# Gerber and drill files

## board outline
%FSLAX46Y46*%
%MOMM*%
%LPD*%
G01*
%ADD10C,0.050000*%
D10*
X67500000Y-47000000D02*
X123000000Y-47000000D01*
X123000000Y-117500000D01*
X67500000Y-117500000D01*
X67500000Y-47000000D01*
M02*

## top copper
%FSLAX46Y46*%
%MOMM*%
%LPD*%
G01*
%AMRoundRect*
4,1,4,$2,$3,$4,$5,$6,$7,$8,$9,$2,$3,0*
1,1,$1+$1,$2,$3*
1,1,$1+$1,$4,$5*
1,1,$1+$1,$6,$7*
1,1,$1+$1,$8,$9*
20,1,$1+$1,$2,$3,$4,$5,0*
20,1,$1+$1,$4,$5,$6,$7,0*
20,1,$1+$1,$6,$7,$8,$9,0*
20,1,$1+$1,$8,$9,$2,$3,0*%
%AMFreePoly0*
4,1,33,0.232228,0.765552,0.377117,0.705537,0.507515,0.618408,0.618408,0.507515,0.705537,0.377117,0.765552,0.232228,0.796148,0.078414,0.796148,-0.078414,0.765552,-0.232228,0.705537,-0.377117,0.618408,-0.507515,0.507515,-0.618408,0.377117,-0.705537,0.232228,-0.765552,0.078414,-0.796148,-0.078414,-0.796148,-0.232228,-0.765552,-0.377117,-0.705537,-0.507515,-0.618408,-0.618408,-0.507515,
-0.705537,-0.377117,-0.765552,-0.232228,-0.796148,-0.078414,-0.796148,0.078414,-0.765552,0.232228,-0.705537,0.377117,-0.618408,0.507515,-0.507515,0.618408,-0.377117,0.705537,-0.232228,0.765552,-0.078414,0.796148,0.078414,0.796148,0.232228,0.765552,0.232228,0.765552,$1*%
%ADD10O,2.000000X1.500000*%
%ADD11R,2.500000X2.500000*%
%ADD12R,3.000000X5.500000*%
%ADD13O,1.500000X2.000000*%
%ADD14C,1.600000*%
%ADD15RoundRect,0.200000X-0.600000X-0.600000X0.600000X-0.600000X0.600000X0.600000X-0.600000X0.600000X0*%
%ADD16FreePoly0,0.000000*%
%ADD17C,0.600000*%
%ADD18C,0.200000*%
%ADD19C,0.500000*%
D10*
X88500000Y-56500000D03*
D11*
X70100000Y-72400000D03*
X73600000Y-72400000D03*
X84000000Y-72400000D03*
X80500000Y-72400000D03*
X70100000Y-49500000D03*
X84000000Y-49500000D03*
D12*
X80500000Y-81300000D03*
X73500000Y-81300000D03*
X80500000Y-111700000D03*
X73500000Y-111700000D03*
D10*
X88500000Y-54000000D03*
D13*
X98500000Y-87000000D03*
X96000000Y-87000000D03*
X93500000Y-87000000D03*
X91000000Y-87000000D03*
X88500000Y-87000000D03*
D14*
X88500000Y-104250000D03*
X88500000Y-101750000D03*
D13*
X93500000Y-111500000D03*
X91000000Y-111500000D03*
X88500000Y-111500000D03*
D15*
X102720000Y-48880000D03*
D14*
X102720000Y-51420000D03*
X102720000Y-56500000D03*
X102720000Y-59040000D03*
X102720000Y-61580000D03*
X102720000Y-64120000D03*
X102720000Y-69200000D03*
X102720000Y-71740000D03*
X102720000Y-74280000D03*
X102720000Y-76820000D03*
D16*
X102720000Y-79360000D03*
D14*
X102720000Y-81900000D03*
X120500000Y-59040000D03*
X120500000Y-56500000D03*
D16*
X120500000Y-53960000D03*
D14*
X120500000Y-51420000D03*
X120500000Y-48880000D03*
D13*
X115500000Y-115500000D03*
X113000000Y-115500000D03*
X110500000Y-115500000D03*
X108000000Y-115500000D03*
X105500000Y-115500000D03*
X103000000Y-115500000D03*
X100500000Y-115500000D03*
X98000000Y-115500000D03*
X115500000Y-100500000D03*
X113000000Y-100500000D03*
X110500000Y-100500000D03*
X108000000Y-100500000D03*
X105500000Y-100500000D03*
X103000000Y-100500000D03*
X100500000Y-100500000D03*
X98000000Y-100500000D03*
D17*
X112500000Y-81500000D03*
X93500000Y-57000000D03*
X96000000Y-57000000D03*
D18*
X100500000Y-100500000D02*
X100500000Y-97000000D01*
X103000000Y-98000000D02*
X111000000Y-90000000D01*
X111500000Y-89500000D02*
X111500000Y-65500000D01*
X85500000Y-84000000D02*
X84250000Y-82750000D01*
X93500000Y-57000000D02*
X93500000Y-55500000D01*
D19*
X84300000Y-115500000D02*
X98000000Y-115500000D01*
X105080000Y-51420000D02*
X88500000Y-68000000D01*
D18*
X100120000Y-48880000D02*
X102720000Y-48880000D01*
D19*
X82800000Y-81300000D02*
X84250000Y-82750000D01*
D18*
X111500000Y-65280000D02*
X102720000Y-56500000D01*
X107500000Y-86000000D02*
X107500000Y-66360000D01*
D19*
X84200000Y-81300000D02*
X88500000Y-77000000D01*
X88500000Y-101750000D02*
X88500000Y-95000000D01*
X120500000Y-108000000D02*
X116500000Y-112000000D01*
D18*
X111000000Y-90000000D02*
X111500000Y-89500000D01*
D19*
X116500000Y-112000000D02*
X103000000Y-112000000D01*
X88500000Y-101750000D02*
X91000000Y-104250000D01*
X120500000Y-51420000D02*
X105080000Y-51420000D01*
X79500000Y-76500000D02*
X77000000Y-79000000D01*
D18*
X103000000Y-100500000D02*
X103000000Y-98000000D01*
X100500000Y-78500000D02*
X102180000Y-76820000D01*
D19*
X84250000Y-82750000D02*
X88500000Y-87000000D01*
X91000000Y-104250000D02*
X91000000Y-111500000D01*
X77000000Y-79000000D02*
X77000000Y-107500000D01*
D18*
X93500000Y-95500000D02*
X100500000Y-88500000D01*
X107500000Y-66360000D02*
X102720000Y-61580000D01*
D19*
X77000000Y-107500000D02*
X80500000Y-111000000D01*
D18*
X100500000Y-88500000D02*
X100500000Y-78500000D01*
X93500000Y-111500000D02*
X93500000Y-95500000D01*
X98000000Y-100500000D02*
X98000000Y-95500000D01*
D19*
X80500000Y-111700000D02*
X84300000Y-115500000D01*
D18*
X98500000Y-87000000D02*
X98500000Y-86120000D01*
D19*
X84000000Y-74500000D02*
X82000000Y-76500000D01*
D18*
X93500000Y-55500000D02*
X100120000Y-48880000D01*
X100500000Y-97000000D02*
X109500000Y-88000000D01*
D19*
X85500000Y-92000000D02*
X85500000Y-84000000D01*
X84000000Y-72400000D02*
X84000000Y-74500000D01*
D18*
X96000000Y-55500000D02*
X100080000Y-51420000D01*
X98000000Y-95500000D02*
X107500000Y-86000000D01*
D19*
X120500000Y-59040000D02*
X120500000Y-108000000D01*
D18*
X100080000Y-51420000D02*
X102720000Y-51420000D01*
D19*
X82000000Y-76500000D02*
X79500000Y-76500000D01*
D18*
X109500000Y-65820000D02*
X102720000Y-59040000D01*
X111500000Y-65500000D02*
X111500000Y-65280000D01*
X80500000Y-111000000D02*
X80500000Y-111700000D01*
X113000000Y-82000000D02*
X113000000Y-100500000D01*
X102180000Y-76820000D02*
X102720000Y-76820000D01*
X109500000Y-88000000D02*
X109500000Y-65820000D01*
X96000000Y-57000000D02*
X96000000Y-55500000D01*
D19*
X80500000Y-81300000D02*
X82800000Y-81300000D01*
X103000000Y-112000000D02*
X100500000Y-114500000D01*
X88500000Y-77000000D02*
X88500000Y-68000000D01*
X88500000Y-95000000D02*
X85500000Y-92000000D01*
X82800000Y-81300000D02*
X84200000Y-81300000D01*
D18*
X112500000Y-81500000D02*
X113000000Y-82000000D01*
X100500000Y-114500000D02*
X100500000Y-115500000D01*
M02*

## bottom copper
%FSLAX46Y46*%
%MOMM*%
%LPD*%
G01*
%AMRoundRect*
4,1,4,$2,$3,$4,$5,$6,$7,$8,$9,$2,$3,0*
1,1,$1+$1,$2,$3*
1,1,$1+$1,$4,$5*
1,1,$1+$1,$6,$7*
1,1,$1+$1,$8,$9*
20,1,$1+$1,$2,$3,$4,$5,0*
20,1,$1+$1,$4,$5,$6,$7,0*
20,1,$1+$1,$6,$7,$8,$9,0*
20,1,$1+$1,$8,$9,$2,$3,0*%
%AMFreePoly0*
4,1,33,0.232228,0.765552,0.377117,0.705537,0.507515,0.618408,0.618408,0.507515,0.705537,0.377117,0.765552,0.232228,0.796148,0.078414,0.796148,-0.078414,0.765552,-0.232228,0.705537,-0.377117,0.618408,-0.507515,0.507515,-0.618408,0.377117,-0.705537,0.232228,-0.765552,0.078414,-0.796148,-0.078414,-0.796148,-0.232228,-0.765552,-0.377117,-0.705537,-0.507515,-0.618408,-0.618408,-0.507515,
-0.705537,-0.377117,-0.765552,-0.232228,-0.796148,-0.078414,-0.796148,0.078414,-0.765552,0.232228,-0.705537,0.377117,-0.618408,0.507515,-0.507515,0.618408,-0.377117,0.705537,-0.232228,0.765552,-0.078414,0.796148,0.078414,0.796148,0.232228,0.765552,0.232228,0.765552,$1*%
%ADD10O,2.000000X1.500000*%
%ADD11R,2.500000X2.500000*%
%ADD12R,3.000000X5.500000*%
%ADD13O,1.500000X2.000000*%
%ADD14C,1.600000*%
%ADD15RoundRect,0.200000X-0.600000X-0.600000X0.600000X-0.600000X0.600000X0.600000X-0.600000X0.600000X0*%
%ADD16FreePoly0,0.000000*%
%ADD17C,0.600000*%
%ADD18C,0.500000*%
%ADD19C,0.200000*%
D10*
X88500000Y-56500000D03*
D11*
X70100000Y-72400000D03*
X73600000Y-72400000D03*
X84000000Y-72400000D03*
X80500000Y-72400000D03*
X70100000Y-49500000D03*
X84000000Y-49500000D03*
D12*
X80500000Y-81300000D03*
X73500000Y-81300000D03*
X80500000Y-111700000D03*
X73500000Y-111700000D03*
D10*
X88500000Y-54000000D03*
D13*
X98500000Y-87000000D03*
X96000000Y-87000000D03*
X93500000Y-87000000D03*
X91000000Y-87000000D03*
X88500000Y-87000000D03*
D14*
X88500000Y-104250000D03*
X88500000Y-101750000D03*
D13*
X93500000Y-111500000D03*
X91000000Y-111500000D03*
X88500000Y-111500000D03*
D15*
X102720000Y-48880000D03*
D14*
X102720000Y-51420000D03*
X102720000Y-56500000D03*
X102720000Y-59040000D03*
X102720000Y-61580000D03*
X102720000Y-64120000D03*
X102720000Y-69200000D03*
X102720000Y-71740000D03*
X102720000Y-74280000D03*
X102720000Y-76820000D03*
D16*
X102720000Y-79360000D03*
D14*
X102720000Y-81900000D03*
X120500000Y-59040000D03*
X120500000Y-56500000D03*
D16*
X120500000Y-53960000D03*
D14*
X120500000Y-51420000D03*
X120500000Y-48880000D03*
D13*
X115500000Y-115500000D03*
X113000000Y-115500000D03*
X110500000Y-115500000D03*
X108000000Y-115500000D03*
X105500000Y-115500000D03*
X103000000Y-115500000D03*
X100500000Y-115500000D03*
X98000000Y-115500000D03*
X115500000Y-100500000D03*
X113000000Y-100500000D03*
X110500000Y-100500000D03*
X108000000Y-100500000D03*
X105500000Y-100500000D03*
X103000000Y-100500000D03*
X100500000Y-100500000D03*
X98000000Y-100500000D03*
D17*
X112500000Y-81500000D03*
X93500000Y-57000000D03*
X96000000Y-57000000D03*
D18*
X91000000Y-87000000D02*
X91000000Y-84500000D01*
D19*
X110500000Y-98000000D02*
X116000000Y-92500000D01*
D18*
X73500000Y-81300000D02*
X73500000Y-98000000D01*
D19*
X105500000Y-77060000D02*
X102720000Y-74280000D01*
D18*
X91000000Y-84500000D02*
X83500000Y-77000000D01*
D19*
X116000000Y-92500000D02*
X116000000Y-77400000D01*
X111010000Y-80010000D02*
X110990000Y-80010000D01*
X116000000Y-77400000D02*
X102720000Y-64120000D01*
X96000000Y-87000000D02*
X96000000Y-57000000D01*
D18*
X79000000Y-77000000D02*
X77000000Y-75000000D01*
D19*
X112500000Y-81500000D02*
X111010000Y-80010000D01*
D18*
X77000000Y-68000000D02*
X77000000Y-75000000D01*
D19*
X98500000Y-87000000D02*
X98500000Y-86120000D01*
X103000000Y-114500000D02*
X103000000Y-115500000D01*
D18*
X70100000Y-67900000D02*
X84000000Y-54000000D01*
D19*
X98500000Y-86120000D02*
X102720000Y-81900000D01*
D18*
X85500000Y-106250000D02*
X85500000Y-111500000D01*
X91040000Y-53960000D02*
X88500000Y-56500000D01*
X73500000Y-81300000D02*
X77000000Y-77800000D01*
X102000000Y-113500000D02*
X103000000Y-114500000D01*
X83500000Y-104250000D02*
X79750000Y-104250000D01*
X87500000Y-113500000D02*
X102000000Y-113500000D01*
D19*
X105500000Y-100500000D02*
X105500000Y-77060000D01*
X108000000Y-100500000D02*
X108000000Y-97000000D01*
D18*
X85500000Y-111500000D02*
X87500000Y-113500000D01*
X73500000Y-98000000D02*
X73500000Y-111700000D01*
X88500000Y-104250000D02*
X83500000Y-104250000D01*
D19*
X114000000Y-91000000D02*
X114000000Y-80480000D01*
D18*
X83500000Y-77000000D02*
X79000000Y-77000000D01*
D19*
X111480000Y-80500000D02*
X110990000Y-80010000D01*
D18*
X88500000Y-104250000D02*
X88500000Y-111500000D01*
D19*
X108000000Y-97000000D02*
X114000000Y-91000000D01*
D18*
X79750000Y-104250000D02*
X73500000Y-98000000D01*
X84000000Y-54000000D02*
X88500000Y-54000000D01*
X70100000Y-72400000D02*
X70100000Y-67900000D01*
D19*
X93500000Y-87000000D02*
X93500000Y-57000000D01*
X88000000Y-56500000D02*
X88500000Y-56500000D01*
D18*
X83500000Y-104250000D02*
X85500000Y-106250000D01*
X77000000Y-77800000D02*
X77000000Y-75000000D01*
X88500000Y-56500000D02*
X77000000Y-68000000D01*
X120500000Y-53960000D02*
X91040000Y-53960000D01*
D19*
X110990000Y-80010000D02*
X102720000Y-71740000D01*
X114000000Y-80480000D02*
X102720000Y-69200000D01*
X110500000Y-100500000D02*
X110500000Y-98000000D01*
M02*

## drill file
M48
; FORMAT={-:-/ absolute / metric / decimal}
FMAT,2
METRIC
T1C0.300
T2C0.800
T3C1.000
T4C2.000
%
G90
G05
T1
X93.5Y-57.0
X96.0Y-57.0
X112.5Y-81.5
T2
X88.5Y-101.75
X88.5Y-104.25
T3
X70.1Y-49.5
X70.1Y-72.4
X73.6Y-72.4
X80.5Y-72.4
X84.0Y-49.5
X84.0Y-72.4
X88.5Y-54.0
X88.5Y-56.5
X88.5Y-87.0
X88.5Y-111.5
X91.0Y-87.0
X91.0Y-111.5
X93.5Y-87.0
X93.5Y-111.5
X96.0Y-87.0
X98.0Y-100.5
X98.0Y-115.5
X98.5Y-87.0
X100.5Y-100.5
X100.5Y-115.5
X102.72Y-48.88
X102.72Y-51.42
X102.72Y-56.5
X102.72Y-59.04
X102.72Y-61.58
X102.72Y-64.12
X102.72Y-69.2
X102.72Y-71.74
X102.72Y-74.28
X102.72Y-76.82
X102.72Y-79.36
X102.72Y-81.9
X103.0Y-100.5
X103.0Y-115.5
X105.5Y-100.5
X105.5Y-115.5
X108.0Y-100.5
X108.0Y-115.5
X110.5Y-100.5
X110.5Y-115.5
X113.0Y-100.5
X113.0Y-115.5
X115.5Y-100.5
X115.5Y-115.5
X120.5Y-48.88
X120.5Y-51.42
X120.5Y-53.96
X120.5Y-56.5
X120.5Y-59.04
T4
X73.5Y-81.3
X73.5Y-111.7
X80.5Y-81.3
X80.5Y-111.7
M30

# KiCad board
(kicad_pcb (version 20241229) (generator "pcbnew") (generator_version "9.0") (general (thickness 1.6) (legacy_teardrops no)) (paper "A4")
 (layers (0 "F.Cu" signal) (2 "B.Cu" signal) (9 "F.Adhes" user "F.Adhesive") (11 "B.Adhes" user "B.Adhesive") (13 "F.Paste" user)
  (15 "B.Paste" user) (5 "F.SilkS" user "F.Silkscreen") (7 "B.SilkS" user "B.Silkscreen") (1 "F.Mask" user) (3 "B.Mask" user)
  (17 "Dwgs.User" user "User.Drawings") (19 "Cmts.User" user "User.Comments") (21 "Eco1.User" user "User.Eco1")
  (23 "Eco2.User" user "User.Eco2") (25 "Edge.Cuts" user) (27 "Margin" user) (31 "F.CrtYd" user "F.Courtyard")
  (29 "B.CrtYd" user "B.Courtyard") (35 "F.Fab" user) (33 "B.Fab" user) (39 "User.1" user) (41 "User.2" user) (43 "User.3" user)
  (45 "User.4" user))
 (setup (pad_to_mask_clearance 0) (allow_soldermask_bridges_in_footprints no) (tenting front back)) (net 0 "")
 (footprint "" (layer "F.Cu") (at 88.5 56.5 90)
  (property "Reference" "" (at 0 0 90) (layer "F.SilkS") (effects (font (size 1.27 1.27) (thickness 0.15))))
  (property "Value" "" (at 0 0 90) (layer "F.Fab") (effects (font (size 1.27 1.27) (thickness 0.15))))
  (pad "2" thru_hole oval (at 0 0 90) (size 1.5 2) (drill 1) (layers "*.Cu" "*.Mask") (remove_unused_layers no)))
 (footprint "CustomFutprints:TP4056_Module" (layer "F.Cu") (at 77.8 61.7 180)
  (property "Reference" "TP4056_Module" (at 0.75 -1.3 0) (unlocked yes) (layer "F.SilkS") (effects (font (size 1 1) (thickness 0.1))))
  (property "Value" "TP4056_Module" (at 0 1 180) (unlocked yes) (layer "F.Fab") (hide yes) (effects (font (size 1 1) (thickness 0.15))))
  (pad "1" thru_hole rect (at 7.7 -10.7 180) (size 2.5 2.5) (drill 1) (layers "*.Cu" "*.Mask") (remove_unused_layers no))
  (pad "2" thru_hole rect (at 4.2 -10.7 180) (size 2.5 2.5) (drill 1) (layers "*.Cu" "*.Mask") (remove_unused_layers no)
   (thermal_bridge_angle 45))
  (pad "3" thru_hole rect (at -6.2 -10.7 180) (size 2.5 2.5) (drill 1) (layers "*.Cu" "*.Mask") (remove_unused_layers no)
   (thermal_bridge_angle 45))
  (pad "4" thru_hole rect (at -2.7 -10.7 180) (size 2.5 2.5) (drill 1) (layers "*.Cu" "*.Mask") (remove_unused_layers no)
   (thermal_bridge_angle 45))
  (pad "5" thru_hole rect (at 7.7 12.2 180) (size 2.5 2.5) (drill 1) (layers "*.Cu" "*.Mask") (remove_unused_layers no)
   (thermal_bridge_angle 45))
  (pad "6" thru_hole rect (at -6.2 12.2 180) (size 2.5 2.5) (drill 1) (layers "*.Cu" "*.Mask") (remove_unused_layers no)
   (thermal_bridge_angle 45)))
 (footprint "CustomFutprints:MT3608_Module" (layer "F.Cu") (at 78.5 88)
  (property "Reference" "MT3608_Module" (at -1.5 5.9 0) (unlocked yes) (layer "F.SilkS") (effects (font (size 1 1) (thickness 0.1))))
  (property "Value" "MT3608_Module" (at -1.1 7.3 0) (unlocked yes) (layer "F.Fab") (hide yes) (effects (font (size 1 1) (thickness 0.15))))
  (pad "1" thru_hole rect (at 2 -6.7) (size 3 5.5) (drill 2) (layers "*.Cu" "*.Mask") (remove_unused_layers no) (thermal_bridge_angle 45))
  (pad "2" thru_hole rect (at -5 -6.7) (size 3 5.5) (drill 2) (layers "*.Cu" "*.Mask") (remove_unused_layers no) (thermal_bridge_angle 45))
  (pad "3" thru_hole rect (at 2 23.7) (size 3 5.5) (drill 2) (layers "*.Cu" "*.Mask") (remove_unused_layers no) (thermal_bridge_angle 45))
  (pad "4" thru_hole rect (at -5 23.7) (size 3 5.5) (drill 2) (layers "*.Cu" "*.Mask") (remove_unused_layers no) (thermal_bridge_angle 45)))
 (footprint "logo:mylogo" (layer "F.Cu") (at 93.5 66.5)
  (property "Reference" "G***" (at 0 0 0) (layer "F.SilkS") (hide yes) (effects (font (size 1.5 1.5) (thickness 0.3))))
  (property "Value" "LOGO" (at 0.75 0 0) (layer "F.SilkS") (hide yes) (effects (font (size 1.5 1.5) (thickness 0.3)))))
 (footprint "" (layer "F.Cu") (at 88.5 54 90)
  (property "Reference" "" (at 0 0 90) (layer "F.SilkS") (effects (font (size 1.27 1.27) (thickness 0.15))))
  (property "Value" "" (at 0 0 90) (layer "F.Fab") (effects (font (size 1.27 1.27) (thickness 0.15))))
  (pad "1" thru_hole oval (at 0 0 90) (size 1.5 2) (drill 1) (layers "*.Cu" "*.Mask") (remove_unused_layers no)))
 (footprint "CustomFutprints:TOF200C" (layer "F.Cu") (at 95.3 90.6)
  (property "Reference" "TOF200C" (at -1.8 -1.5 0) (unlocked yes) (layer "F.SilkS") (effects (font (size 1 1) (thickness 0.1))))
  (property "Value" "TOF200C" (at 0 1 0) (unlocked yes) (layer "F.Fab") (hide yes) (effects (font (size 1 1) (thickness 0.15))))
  (pad "1" thru_hole oval (at 3.2 -3.6) (size 1.5 2) (drill 1) (layers "*.Cu" "*.Mask") (remove_unused_layers no))
  (pad "2" thru_hole oval (at 0.7 -3.6) (size 1.5 2) (drill 1) (layers "*.Cu" "*.Mask") (remove_unused_layers no))
  (pad "3" thru_hole oval (at -1.8 -3.6) (size 1.5 2) (drill 1) (layers "*.Cu" "*.Mask") (remove_unused_layers no))
  (pad "4" thru_hole oval (at -4.3 -3.6) (size 1.5 2) (drill 1) (layers "*.Cu" "*.Mask") (remove_unused_layers no))
  (pad "5" thru_hole oval (at -6.8 -3.6) (size 1.5 2) (drill 1) (layers "*.Cu" "*.Mask") (remove_unused_layers no)))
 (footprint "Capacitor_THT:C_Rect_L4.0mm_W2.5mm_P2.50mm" (layer "F.Cu") (at 88.5 104.25 90)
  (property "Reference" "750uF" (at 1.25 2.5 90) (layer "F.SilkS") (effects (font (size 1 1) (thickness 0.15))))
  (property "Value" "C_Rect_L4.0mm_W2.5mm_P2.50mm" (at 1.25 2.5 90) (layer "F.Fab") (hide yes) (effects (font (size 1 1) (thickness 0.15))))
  (pad "1" thru_hole circle (at 0 0 90) (size 1.6 1.6) (drill 0.8) (layers "*.Cu" "*.Mask") (remove_unused_layers no))
  (pad "2" thru_hole circle (at 2.5 0 90) (size 1.6 1.6) (drill 0.8) (layers "*.Cu" "*.Mask") (remove_unused_layers no)))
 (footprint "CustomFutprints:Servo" (layer "F.Cu") (at 90.95 114.2)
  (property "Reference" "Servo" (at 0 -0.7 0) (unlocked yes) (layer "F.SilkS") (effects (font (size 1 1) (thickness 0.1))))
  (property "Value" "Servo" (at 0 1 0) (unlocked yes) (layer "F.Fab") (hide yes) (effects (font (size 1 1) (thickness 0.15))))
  (pad "1" thru_hole oval (at 2.55 -2.7) (size 1.5 2) (drill 1) (layers "*.Cu" "*.Mask") (remove_unused_layers no))
  (pad "2" thru_hole oval (at 0.05 -2.7) (size 1.5 2) (drill 1) (layers "*.Cu" "*.Mask") (remove_unused_layers no))
  (pad "3" thru_hole oval (at -2.45 -2.7) (size 1.5 2) (drill 1) (layers "*.Cu" "*.Mask") (remove_unused_layers no)))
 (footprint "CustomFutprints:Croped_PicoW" (layer "F.Cu") (at 112.07 67.38)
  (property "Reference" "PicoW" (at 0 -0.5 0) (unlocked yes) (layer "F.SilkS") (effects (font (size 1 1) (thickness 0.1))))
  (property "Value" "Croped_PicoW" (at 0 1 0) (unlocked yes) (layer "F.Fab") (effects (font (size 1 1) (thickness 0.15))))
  (pad "1" thru_hole roundrect (at -9.35 -18.5) (size 1.6 1.6) (drill 1) (layers "*.Cu" "*.Mask") (remove_unused_layers no)
   (roundrect_rratio 0.125))
  (pad "2" thru_hole circle (at -9.35 -15.96) (size 1.6 1.6) (drill 1) (layers "*.Cu" "*.Mask") (remove_unused_layers no))
  (pad "4" thru_hole circle (at -9.35 -10.88) (size 1.6 1.6) (drill 1) (layers "*.Cu" "*.Mask") (remove_unused_layers no))
  (pad "5" thru_hole circle (at -9.35 -8.34) (size 1.6 1.6) (drill 1) (layers "*.Cu" "*.Mask") (remove_unused_layers no))
  (pad "6" thru_hole circle (at -9.35 -5.8) (size 1.6 1.6) (drill 1) (layers "*.Cu" "*.Mask") (remove_unused_layers no))
  (pad "7" thru_hole circle (at -9.35 -3.26) (size 1.6 1.6) (drill 1) (layers "*.Cu" "*.Mask") (remove_unused_layers no))
  (pad "9" thru_hole circle (at -9.35 1.82) (size 1.6 1.6) (drill 1) (layers "*.Cu" "*.Mask") (remove_unused_layers no))
  (pad "10" thru_hole circle (at -9.35 4.36) (size 1.6 1.6) (drill 1) (layers "*.Cu" "*.Mask") (remove_unused_layers no))
  (pad "11" thru_hole circle (at -9.35 6.9) (size 1.6 1.6) (drill 1) (layers "*.Cu" "*.Mask") (remove_unused_layers no))
  (pad "12" thru_hole circle (at -9.35 9.44) (size 1.6 1.6) (drill 1) (layers "*.Cu" "*.Mask") (remove_unused_layers no))
  (pad "13" thru_hole custom (at -9.35 11.98) (size 1.6 1.6) (drill 1) (layers "*.Cu" "*.Mask") (remove_unused_layers no)
   (options (clearance outline) (anchor circle)) (primitives))
  (pad "14" thru_hole circle (at -9.35 14.52) (size 1.6 1.6) (drill 1) (layers "*.Cu" "*.Mask") (remove_unused_layers no))
  (pad "36" thru_hole circle (at 8.43 -8.34) (size 1.6 1.6) (drill 1) (layers "*.Cu" "*.Mask") (remove_unused_layers no))
  (pad "37" thru_hole circle (at 8.43 -10.88) (size 1.6 1.6) (drill 1) (layers "*.Cu" "*.Mask") (remove_unused_layers no))
  (pad "38" thru_hole custom (at 8.43 -13.42) (size 1.6 1.6) (drill 1) (layers "*.Cu" "*.Mask") (remove_unused_layers no)
   (options (clearance outline) (anchor circle)) (primitives))
  (pad "39" thru_hole circle (at 8.43 -15.96) (size 1.6 1.6) (drill 1) (layers "*.Cu" "*.Mask") (remove_unused_layers no))
  (pad "40" thru_hole circle (at 8.43 -18.5) (size 1.6 1.6) (drill 1) (layers "*.Cu" "*.Mask") (remove_unused_layers no)))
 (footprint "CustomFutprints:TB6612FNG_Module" (layer "F.Cu") (at 107.8 106.2)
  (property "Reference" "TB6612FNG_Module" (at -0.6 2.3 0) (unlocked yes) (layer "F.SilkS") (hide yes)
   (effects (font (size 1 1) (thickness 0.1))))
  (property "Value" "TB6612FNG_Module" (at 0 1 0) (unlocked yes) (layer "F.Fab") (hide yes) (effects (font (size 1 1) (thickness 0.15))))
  (pad "1" thru_hole oval (at 7.7 9.3) (size 1.5 2) (drill 1) (layers "*.Cu" "*.Mask") (remove_unused_layers no))
  (pad "2" thru_hole oval (at 5.2 9.3) (size 1.5 2) (drill 1) (layers "*.Cu" "*.Mask") (remove_unused_layers no))
  (pad "3" thru_hole oval (at 2.7 9.3) (size 1.5 2) (drill 1) (layers "*.Cu" "*.Mask") (remove_unused_layers no))
  (pad "4" thru_hole oval (at 0.2 9.3) (size 1.5 2) (drill 1) (layers "*.Cu" "*.Mask") (remove_unused_layers no))
  (pad "5" thru_hole oval (at -2.3 9.3) (size 1.5 2) (drill 1) (layers "*.Cu" "*.Mask") (remove_unused_layers no))
  (pad "6" thru_hole oval (at -4.8 9.3) (size 1.5 2) (drill 1) (layers "*.Cu" "*.Mask") (remove_unused_layers no))
  (pad "7" thru_hole oval (at -7.3 9.3) (size 1.5 2) (drill 1) (layers "*.Cu" "*.Mask") (remove_unused_layers no))
  (pad "8" thru_hole oval (at -9.8 9.3) (size 1.5 2) (drill 1) (layers "*.Cu" "*.Mask") (remove_unused_layers no))
  (pad "9" thru_hole oval (at 7.7 -5.7) (size 1.5 2) (drill 1) (layers "*.Cu" "*.Mask") (remove_unused_layers no))
  (pad "10" thru_hole oval (at 5.2 -5.7) (size 1.5 2) (drill 1) (layers "*.Cu" "*.Mask") (remove_unused_layers no))
  (pad "11" thru_hole oval (at 2.7 -5.7) (size 1.5 2) (drill 1) (layers "*.Cu" "*.Mask") (remove_unused_layers no))
  (pad "12" thru_hole oval (at 0.2 -5.7) (size 1.5 2) (drill 1) (layers "*.Cu" "*.Mask") (remove_unused_layers no))
  (pad "13" thru_hole oval (at -2.3 -5.7) (size 1.5 2) (drill 1) (layers "*.Cu" "*.Mask") (remove_unused_layers no))
  (pad "14" thru_hole oval (at -4.8 -5.7) (size 1.5 2) (drill 1) (layers "*.Cu" "*.Mask") (remove_unused_layers no))
  (pad "15" thru_hole oval (at -7.3 -5.7) (size 1.5 2) (drill 1) (layers "*.Cu" "*.Mask") (remove_unused_layers no))
  (pad "16" thru_hole oval (at -9.8 -5.7) (size 1.5 2) (drill 1) (layers "*.Cu" "*.Mask") (remove_unused_layers no)))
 (gr_rect (start 67.5 47) (end 123 117.5) (stroke (width 0.05) (type solid)) (fill no) (layer "Edge.Cuts"))
 (segment (start 100.5 100.5) (end 100.5 97) (width 0.2) (layer "F.Cu") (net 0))
 (segment (start 103 98) (end 111 90) (width 0.2) (layer "F.Cu") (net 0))
 (segment (start 111.5 89.5) (end 111.5 65.5) (width 0.2) (layer "F.Cu") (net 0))
 (segment (start 85.5 84) (end 84.25 82.75) (width 0.2) (layer "F.Cu") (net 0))
 (segment (start 93.5 57) (end 93.5 55.5) (width 0.2) (layer "F.Cu") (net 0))
 (segment (start 84.3 115.5) (end 98 115.5) (width 0.5) (layer "F.Cu") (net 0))
 (segment (start 105.08 51.42) (end 88.5 68) (width 0.5) (layer "F.Cu") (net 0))
 (segment (start 100.12 48.88) (end 102.72 48.88) (width 0.2) (layer "F.Cu") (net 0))
 (segment (start 82.8 81.3) (end 84.25 82.75) (width 0.5) (layer "F.Cu") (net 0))
 (segment (start 111.5 65.28) (end 102.72 56.5) (width 0.2) (layer "F.Cu") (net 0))
 (segment (start 107.5 86) (end 107.5 66.36) (width 0.2) (layer "F.Cu") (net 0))
 (segment (start 84.2 81.3) (end 88.5 77) (width 0.5) (layer "F.Cu") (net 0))
 (segment (start 88.5 101.75) (end 88.5 95) (width 0.5) (layer "F.Cu") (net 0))
 (segment (start 120.5 108) (end 116.5 112) (width 0.5) (layer "F.Cu") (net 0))
 (segment (start 111 90) (end 111.5 89.5) (width 0.2) (layer "F.Cu") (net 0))
 (segment (start 116.5 112) (end 103 112) (width 0.5) (layer "F.Cu") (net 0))
 (segment (start 88.5 101.75) (end 91 104.25) (width 0.5) (layer "F.Cu") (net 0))
 (segment (start 120.5 51.42) (end 105.08 51.42) (width 0.5) (layer "F.Cu") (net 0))
 (segment (start 79.5 76.5) (end 77 79) (width 0.5) (layer "F.Cu") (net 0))
 (segment (start 103 100.5) (end 103 98) (width 0.2) (layer "F.Cu") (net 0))
 (segment (start 100.5 78.5) (end 102.18 76.82) (width 0.2) (layer "F.Cu") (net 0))
 (segment (start 84.25 82.75) (end 88.5 87) (width 0.5) (layer "F.Cu") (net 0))
 (segment (start 91 104.25) (end 91 111.5) (width 0.5) (layer "F.Cu") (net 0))
 (segment (start 77 79) (end 77 107.5) (width 0.5) (layer "F.Cu") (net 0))
 (segment (start 93.5 95.5) (end 100.5 88.5) (width 0.2) (layer "F.Cu") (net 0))
 (segment (start 107.5 66.36) (end 102.72 61.58) (width 0.2) (layer "F.Cu") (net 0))
 (segment (start 77 107.5) (end 80.5 111) (width 0.5) (layer "F.Cu") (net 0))
 (segment (start 100.5 88.5) (end 100.5 78.5) (width 0.2) (layer "F.Cu") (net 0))
 (segment (start 93.5 111.5) (end 93.5 95.5) (width 0.2) (layer "F.Cu") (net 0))
 (segment (start 98 100.5) (end 98 95.5) (width 0.2) (layer "F.Cu") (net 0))
 (segment (start 80.5 111.7) (end 84.3 115.5) (width 0.5) (layer "F.Cu") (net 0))
 (segment (start 98.5 87) (end 98.5 86.12) (width 0.2) (layer "F.Cu") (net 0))
 (segment (start 84 74.5) (end 82 76.5) (width 0.5) (layer "F.Cu") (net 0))
 (segment (start 93.5 55.5) (end 100.12 48.88) (width 0.2) (layer "F.Cu") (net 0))
 (segment (start 100.5 97) (end 109.5 88) (width 0.2) (layer "F.Cu") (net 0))
 (segment (start 85.5 92) (end 85.5 84) (width 0.5) (layer "F.Cu") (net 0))
 (segment (start 84 72.4) (end 84 74.5) (width 0.5) (layer "F.Cu") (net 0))
 (segment (start 96 55.5) (end 100.08 51.42) (width 0.2) (layer "F.Cu") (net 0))
 (segment (start 98 95.5) (end 107.5 86) (width 0.2) (layer "F.Cu") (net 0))
 (segment (start 120.5 59.04) (end 120.5 108) (width 0.5) (layer "F.Cu") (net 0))
 (segment (start 100.08 51.42) (end 102.72 51.42) (width 0.2) (layer "F.Cu") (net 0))
 (segment (start 82 76.5) (end 79.5 76.5) (width 0.5) (layer "F.Cu") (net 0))
 (segment (start 109.5 65.82) (end 102.72 59.04) (width 0.2) (layer "F.Cu") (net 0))
 (segment (start 111.5 65.5) (end 111.5 65.28) (width 0.2) (layer "F.Cu") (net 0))
 (segment (start 80.5 111) (end 80.5 111.7) (width 0.2) (layer "F.Cu") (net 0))
 (segment (start 113 82) (end 113 100.5) (width 0.2) (layer "F.Cu") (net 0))
 (segment (start 102.18 76.82) (end 102.72 76.82) (width 0.2) (layer "F.Cu") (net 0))
 (segment (start 109.5 88) (end 109.5 65.82) (width 0.2) (layer "F.Cu") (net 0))
 (segment (start 96 57) (end 96 55.5) (width 0.2) (layer "F.Cu") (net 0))
 (segment (start 80.5 81.3) (end 82.8 81.3) (width 0.5) (layer "F.Cu") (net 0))
 (segment (start 103 112) (end 100.5 114.5) (width 0.5) (layer "F.Cu") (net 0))
 (segment (start 88.5 77) (end 88.5 68) (width 0.5) (layer "F.Cu") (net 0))
 (segment (start 88.5 95) (end 85.5 92) (width 0.5) (layer "F.Cu") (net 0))
 (segment (start 82.8 81.3) (end 84.2 81.3) (width 0.5) (layer "F.Cu") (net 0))
 (segment (start 112.5 81.5) (end 113 82) (width 0.2) (layer "F.Cu") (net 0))
 (segment (start 100.5 114.5) (end 100.5 115.5) (width 0.2) (layer "F.Cu") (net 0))
 (via (at 112.5 81.5) (size 0.6) (drill 0.3) (layers "F.Cu" "B.Cu") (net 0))
 (via (at 93.5 57) (size 0.6) (drill 0.3) (layers "F.Cu" "B.Cu") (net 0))
 (via (at 96 57) (size 0.6) (drill 0.3) (layers "F.Cu" "B.Cu") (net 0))
 (segment (start 91 87) (end 91 84.5) (width 0.5) (layer "B.Cu") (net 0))
 (segment (start 110.5 98) (end 116 92.5) (width 0.2) (layer "B.Cu") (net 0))
 (segment (start 73.5 81.3) (end 73.5 98) (width 0.5) (layer "B.Cu") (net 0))
 (segment (start 105.5 77.06) (end 102.72 74.28) (width 0.2) (layer "B.Cu") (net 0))
 (segment (start 91 84.5) (end 83.5 77) (width 0.5) (layer "B.Cu") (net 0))
 (segment (start 116 92.5) (end 116 77.4) (width 0.2) (layer "B.Cu") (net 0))
 (segment (start 111.01 80.01) (end 110.99 80.01) (width 0.2) (layer "B.Cu") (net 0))
 (segment (start 116 77.4) (end 102.72 64.12) (width 0.2) (layer "B.Cu") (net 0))
 (segment (start 96 87) (end 96 57) (width 0.2) (layer "B.Cu") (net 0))
 (segment (start 79 77) (end 77 75) (width 0.5) (layer "B.Cu") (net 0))
 (segment (start 112.5 81.5) (end 111.01 80.01) (width 0.2) (layer "B.Cu") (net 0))
 (segment (start 77 68) (end 77 75) (width 0.5) (layer "B.Cu") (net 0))
 (segment (start 98.5 87) (end 98.5 86.12) (width 0.2) (layer "B.Cu") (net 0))
 (segment (start 103 114.5) (end 103 115.5) (width 0.2) (layer "B.Cu") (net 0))
 (segment (start 70.1 67.9) (end 84 54) (width 0.5) (layer "B.Cu") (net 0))
 (segment (start 98.5 86.12) (end 102.72 81.9) (width 0.2) (layer "B.Cu") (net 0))
 (segment (start 85.5 106.25) (end 85.5 111.5) (width 0.5) (layer "B.Cu") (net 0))
 (segment (start 91.04 53.96) (end 88.5 56.5) (width 0.5) (layer "B.Cu") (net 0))
 (segment (start 73.5 81.3) (end 77 77.8) (width 0.5) (layer "B.Cu") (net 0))
 (segment (start 102 113.5) (end 103 114.5) (width 0.5) (layer "B.Cu") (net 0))
 (segment (start 83.5 104.25) (end 79.75 104.25) (width 0.5) (layer "B.Cu") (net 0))
 (segment (start 87.5 113.5) (end 102 113.5) (width 0.5) (layer "B.Cu") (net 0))
 (segment (start 105.5 100.5) (end 105.5 77.06) (width 0.2) (layer "B.Cu") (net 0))
 (segment (start 108 100.5) (end 108 97) (width 0.2) (layer "B.Cu") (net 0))
 (segment (start 85.5 111.5) (end 87.5 113.5) (width 0.5) (layer "B.Cu") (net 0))
 (segment (start 73.5 98) (end 73.5 111.7) (width 0.5) (layer "B.Cu") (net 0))
 (segment (start 88.5 104.25) (end 83.5 104.25) (width 0.5) (layer "B.Cu") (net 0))
 (segment (start 114 91) (end 114 80.48) (width 0.2) (layer "B.Cu") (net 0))
 (segment (start 83.5 77) (end 79 77) (width 0.5) (layer "B.Cu") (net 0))
 (segment (start 111.48 80.5) (end 110.99 80.01) (width 0.2) (layer "B.Cu") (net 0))
 (segment (start 88.5 104.25) (end 88.5 111.5) (width 0.5) (layer "B.Cu") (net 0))
 (segment (start 108 97) (end 114 91) (width 0.2) (layer "B.Cu") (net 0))
 (segment (start 79.75 104.25) (end 73.5 98) (width 0.5) (layer "B.Cu") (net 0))
 (segment (start 84 54) (end 88.5 54) (width 0.5) (layer "B.Cu") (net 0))
 (segment (start 70.1 72.4) (end 70.1 67.9) (width 0.5) (layer "B.Cu") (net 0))
 (segment (start 93.5 87) (end 93.5 57) (width 0.2) (layer "B.Cu") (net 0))
 (segment (start 88 56.5) (end 88.5 56.5) (width 0.2) (layer "B.Cu") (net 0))
 (segment (start 83.5 104.25) (end 85.5 106.25) (width 0.5) (layer "B.Cu") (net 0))
 (segment (start 77 77.8) (end 77 75) (width 0.5) (layer "B.Cu") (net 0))
 (segment (start 88.5 56.5) (end 77 68) (width 0.5) (layer "B.Cu") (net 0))
 (segment (start 120.5 53.96) (end 91.04 53.96) (width 0.5) (layer "B.Cu") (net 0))
 (segment (start 110.99 80.01) (end 102.72 71.74) (width 0.2) (layer "B.Cu") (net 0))
 (segment (start 114 80.48) (end 102.72 69.2) (width 0.2) (layer "B.Cu") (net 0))
 (segment (start 110.5 100.5) (end 110.5 98) (width 0.2) (layer "B.Cu") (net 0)))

